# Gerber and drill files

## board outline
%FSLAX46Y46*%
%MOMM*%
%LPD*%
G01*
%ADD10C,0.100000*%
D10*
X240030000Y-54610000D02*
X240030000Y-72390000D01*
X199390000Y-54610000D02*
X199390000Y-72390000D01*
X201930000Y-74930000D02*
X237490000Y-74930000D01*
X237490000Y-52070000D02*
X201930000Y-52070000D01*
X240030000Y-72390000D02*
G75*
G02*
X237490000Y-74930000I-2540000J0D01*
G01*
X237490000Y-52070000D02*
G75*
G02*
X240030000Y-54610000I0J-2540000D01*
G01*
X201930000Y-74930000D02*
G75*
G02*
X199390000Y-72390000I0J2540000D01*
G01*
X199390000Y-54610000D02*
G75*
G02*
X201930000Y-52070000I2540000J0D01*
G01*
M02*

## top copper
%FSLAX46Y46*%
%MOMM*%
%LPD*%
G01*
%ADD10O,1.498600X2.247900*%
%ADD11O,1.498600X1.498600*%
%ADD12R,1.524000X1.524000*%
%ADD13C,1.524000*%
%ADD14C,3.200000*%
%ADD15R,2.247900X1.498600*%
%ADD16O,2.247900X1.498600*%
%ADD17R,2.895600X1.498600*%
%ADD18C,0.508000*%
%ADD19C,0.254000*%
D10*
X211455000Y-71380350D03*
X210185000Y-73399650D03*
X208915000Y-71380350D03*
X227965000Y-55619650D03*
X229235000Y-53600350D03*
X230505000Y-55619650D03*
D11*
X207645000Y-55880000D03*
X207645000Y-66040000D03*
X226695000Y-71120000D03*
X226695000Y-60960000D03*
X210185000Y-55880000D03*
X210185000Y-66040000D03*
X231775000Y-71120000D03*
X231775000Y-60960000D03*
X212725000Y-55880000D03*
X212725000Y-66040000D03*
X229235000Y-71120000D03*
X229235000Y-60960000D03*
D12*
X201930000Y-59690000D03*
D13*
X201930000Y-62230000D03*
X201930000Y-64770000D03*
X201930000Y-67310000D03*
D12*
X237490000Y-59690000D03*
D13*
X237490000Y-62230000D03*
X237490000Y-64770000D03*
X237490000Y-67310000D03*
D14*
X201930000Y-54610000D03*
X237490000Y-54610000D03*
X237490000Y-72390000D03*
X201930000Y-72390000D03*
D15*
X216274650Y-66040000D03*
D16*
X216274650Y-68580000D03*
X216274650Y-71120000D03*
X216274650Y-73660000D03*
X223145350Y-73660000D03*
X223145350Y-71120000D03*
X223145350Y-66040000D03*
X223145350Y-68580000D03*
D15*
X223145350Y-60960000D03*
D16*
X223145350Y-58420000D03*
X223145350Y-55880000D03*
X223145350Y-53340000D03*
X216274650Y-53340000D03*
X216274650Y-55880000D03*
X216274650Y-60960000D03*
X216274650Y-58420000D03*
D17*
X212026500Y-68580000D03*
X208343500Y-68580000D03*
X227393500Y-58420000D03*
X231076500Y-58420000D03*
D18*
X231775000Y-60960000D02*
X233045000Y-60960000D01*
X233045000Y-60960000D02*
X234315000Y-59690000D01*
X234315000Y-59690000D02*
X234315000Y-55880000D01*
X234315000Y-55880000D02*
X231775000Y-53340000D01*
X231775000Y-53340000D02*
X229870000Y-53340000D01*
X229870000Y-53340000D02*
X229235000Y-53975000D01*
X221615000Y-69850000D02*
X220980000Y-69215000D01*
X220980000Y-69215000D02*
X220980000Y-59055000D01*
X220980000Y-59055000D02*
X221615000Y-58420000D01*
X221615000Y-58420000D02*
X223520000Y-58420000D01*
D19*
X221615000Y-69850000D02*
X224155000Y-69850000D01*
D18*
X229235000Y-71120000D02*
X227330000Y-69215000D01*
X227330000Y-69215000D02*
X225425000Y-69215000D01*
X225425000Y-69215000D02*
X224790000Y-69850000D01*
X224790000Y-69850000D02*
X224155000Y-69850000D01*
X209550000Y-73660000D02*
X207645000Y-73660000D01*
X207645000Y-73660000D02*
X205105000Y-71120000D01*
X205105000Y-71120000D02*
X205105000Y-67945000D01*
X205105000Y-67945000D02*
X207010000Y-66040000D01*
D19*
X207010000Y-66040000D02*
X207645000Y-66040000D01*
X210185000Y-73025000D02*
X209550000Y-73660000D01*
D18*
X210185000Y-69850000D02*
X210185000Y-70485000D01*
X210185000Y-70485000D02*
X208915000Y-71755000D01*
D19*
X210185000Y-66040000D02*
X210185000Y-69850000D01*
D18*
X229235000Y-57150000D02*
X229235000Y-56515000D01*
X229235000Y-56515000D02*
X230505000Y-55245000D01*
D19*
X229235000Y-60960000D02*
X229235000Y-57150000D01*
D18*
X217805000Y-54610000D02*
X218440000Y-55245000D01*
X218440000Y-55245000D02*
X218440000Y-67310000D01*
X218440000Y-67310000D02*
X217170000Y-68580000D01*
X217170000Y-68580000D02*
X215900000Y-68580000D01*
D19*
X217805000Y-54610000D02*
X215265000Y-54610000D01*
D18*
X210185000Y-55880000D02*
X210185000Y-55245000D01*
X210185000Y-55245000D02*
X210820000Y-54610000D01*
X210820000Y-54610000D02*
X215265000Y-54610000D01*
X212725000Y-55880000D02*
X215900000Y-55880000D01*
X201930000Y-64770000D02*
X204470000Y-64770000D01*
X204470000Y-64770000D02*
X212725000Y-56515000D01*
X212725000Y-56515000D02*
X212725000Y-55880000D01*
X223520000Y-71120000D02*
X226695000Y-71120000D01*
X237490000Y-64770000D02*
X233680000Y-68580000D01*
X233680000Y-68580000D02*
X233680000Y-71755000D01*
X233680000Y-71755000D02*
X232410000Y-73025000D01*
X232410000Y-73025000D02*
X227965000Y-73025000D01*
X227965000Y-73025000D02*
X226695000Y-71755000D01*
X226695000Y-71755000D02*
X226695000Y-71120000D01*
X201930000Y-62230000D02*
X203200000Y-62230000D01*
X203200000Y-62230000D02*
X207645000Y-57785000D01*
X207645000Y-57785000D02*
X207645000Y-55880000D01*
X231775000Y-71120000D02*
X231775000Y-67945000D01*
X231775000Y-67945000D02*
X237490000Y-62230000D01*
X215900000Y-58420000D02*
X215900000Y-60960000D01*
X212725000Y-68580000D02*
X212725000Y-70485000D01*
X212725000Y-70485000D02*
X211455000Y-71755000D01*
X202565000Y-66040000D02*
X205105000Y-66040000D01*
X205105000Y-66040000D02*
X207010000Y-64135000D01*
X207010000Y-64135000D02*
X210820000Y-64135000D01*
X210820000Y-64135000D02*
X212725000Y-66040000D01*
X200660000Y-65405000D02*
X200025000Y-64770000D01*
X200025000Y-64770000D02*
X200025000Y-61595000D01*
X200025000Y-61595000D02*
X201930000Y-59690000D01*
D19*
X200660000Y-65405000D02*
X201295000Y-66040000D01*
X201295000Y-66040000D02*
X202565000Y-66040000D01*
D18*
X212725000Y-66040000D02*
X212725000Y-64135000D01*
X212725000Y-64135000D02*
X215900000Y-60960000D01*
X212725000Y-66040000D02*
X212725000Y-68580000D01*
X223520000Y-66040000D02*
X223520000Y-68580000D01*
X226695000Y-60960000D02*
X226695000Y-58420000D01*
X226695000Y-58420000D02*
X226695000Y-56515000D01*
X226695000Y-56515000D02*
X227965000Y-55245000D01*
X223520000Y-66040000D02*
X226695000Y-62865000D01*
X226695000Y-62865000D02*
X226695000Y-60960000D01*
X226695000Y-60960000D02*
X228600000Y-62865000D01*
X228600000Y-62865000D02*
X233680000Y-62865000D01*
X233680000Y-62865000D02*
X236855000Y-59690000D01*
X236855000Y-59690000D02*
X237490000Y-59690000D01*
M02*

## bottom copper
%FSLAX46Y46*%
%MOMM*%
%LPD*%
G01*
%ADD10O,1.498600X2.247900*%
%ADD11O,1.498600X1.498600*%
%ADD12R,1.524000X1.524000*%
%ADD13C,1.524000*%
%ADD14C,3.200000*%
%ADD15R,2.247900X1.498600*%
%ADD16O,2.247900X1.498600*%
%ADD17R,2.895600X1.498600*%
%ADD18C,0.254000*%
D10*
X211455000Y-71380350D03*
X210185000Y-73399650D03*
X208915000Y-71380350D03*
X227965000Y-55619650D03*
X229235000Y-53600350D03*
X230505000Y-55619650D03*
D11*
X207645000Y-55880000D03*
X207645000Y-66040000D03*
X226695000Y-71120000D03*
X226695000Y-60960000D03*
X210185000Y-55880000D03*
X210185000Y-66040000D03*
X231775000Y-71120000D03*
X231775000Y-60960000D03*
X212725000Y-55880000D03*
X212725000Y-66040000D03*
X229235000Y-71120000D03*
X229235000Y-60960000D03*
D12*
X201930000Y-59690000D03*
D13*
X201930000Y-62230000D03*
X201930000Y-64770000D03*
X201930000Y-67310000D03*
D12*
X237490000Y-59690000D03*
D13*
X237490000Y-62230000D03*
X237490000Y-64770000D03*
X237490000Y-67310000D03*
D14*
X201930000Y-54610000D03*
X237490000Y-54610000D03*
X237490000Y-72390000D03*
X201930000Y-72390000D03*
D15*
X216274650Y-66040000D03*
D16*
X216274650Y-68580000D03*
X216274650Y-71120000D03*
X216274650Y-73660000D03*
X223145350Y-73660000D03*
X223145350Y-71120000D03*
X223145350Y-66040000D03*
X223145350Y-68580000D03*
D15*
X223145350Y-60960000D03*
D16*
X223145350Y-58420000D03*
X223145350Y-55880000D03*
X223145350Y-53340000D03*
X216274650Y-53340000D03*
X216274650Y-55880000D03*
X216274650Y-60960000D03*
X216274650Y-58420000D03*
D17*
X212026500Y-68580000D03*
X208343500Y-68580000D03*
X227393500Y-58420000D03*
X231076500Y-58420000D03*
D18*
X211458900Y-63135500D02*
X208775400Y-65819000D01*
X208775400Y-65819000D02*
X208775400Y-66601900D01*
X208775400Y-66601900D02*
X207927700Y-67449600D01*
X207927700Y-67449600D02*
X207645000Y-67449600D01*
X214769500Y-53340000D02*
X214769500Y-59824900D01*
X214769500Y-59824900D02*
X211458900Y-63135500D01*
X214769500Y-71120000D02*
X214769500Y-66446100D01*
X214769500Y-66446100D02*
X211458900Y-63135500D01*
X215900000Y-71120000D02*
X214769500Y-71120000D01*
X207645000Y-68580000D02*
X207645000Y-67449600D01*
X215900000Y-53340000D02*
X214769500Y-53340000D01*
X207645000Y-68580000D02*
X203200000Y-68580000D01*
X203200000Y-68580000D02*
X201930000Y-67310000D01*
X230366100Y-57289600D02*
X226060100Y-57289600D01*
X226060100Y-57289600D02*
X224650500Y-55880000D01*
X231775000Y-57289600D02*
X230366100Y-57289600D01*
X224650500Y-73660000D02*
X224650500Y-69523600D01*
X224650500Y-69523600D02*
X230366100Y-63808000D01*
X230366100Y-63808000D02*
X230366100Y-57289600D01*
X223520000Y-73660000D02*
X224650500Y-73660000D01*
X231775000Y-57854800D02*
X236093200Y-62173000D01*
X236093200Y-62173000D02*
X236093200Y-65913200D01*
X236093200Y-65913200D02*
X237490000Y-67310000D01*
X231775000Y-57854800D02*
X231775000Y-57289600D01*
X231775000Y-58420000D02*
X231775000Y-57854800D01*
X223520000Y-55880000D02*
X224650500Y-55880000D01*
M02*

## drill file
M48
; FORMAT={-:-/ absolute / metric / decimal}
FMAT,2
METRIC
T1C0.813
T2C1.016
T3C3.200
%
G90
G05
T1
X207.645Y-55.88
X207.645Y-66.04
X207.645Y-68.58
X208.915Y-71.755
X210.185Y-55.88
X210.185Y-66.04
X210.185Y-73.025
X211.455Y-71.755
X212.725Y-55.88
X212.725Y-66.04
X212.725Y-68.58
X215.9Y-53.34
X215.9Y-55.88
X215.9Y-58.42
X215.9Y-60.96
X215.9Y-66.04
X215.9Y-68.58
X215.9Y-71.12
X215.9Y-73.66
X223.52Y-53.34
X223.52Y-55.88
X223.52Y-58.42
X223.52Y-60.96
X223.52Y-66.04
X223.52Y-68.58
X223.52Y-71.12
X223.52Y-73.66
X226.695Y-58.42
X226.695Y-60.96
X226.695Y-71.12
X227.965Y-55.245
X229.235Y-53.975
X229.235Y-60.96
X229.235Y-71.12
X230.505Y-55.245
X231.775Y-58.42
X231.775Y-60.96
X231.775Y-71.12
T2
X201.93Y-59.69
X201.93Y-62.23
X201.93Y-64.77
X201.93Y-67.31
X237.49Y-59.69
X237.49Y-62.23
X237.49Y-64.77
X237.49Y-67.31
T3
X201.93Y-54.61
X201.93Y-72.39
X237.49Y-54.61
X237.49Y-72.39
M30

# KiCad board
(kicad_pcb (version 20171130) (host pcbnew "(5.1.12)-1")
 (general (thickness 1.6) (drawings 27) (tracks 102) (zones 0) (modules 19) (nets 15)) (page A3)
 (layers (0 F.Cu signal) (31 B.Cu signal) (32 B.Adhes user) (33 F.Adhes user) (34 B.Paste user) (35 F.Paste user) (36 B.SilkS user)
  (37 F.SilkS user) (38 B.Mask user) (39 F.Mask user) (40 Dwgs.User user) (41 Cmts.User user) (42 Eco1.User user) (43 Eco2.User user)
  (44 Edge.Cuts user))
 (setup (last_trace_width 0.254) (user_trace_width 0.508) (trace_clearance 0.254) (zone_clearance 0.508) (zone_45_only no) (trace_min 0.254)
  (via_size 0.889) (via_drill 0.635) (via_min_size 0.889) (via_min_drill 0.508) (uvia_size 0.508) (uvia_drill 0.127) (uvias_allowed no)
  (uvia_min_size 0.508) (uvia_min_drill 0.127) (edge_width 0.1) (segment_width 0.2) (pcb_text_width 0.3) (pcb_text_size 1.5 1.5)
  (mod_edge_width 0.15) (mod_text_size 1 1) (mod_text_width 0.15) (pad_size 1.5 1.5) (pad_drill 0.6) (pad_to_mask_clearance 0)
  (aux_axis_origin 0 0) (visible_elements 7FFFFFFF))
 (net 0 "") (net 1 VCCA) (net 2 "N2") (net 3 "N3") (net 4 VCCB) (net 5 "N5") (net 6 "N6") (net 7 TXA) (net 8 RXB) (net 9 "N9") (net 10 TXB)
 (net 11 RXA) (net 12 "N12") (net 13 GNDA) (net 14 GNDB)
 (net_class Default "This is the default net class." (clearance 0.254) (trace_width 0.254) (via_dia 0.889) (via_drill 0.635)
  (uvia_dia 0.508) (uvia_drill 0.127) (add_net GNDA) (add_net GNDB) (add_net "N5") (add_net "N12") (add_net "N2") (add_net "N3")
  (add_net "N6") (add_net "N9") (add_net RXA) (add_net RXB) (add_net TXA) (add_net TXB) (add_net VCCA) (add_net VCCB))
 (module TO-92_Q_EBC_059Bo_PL (layer F.Cu) (at 211.455 71.755)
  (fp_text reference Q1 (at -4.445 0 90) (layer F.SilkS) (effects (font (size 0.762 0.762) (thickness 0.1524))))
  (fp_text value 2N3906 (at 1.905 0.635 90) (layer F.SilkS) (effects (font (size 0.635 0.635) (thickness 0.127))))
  (pad 1 thru_hole oval (at 0 0) (size 1.4986 2.2479) (drill 0.8128 (offset 0 -0.37465)) (layers *.Cu *.Mask F.SilkS) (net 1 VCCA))
  (pad 2 thru_hole oval (at -1.27 1.27) (size 1.4986 2.2479) (drill 0.8128 (offset 0 0.37465)) (layers *.Cu *.Mask F.SilkS) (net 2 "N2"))
  (pad 3 thru_hole oval (at -2.54 0) (size 1.4986 2.2479) (drill 0.8128 (offset 0 -0.37465)) (layers *.Cu *.Mask F.SilkS) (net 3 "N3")))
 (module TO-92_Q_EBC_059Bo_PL (layer F.Cu) (at 227.965 55.245 180)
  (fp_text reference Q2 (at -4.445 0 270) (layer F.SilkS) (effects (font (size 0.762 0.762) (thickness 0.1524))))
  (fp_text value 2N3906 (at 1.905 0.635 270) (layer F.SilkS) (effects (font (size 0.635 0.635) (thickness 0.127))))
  (pad 1 thru_hole oval (at 0 0 180) (size 1.4986 2.2479) (drill 0.8128 (offset 0 -0.37465)) (layers *.Cu *.Mask F.SilkS) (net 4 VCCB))
  (pad 2 thru_hole oval (at -1.27 1.27 180) (size 1.4986 2.2479) (drill 0.8128 (offset 0 0.37465)) (layers *.Cu *.Mask F.SilkS) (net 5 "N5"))
  (pad 3 thru_hole oval (at -2.54 0 180) (size 1.4986 2.2479) (drill 0.8128 (offset 0 -0.37465)) (layers *.Cu *.Mask F.SilkS) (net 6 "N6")))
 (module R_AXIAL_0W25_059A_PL (layer F.Cu) (at 207.645 55.88 270) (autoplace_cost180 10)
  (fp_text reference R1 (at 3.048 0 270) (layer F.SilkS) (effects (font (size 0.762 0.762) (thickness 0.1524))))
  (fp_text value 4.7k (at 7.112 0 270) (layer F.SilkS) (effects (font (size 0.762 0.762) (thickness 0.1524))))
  (pad 1 thru_hole oval (at 0 0 270) (size 1.4986 1.4986) (drill 0.8128) (layers *.Cu *.Mask F.SilkS) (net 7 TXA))
  (pad 2 thru_hole oval (at 10.16 0 270) (size 1.4986 1.4986) (drill 0.8128) (layers *.Cu *.Mask F.SilkS) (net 2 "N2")))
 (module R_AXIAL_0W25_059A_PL (layer F.Cu) (at 226.695 71.12 90) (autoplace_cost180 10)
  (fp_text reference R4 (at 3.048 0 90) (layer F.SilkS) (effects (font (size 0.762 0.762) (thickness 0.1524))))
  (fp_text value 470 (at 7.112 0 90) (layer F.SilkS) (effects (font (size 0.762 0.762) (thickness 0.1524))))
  (pad 1 thru_hole oval (at 0 0 90) (size 1.4986 1.4986) (drill 0.8128) (layers *.Cu *.Mask F.SilkS) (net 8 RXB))
  (pad 2 thru_hole oval (at 10.16 0 90) (size 1.4986 1.4986) (drill 0.8128) (layers *.Cu *.Mask F.SilkS) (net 4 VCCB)))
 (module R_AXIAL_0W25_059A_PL (layer F.Cu) (at 210.185 55.88 270) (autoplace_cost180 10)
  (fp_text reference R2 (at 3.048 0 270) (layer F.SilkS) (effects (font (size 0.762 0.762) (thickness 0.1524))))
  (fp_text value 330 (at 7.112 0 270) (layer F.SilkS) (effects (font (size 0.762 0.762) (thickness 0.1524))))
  (pad 1 thru_hole oval (at 0 0 270) (size 1.4986 1.4986) (drill 0.8128) (layers *.Cu *.Mask F.SilkS) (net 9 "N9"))
  (pad 2 thru_hole oval (at 10.16 0 270) (size 1.4986 1.4986) (drill 0.8128) (layers *.Cu *.Mask F.SilkS) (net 3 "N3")))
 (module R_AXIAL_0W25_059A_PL (layer F.Cu) (at 231.775 71.12 90) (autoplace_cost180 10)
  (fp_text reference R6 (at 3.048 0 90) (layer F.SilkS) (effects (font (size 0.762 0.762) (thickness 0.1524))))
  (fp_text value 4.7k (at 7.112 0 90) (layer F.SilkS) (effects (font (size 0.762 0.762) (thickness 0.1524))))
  (pad 1 thru_hole oval (at 0 0 90) (size 1.4986 1.4986) (drill 0.8128) (layers *.Cu *.Mask F.SilkS) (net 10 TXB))
  (pad 2 thru_hole oval (at 10.16 0 90) (size 1.4986 1.4986) (drill 0.8128) (layers *.Cu *.Mask F.SilkS) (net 5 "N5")))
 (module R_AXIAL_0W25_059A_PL (layer F.Cu) (at 212.725 55.88 270) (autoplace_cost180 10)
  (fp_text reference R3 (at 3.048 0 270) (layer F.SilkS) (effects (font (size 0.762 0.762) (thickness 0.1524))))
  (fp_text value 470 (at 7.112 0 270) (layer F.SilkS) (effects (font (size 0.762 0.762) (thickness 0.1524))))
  (pad 1 thru_hole oval (at 0 0 270) (size 1.4986 1.4986) (drill 0.8128) (layers *.Cu *.Mask F.SilkS) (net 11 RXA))
  (pad 2 thru_hole oval (at 10.16 0 270) (size 1.4986 1.4986) (drill 0.8128) (layers *.Cu *.Mask F.SilkS) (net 1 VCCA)))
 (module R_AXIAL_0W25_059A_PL (layer F.Cu) (at 229.235 71.12 90) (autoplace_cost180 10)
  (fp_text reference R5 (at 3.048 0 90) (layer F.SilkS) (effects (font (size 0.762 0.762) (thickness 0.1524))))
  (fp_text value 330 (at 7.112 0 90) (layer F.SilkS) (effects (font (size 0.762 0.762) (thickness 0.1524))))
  (pad 1 thru_hole oval (at 0 0 90) (size 1.4986 1.4986) (drill 0.8128) (layers *.Cu *.Mask F.SilkS) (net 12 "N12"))
  (pad 2 thru_hole oval (at 10.16 0 90) (size 1.4986 1.4986) (drill 0.8128) (layers *.Cu *.Mask F.SilkS) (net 6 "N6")))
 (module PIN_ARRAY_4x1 (layer F.Cu) (at 201.93 63.5 270)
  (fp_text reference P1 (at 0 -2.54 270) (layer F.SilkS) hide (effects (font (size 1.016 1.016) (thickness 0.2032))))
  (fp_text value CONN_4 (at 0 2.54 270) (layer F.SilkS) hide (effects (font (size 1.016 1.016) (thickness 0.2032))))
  (pad 1 thru_hole rect (at -3.81 0 270) (size 1.524 1.524) (drill 1.016) (layers *.Cu *.Mask F.SilkS) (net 1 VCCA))
  (pad 2 thru_hole circle (at -1.27 0 270) (size 1.524 1.524) (drill 1.016) (layers *.Cu *.Mask F.SilkS) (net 7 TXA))
  (pad 3 thru_hole circle (at 1.27 0 270) (size 1.524 1.524) (drill 1.016) (layers *.Cu *.Mask F.SilkS) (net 11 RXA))
  (pad 4 thru_hole circle (at 3.81 0 270) (size 1.524 1.524) (drill 1.016) (layers *.Cu *.Mask F.SilkS) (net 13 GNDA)))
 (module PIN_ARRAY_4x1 (layer F.Cu) (at 237.49 63.5 270)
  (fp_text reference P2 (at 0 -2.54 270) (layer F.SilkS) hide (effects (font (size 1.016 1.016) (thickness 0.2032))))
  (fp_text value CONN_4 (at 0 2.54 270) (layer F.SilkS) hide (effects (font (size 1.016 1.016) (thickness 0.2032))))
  (pad 1 thru_hole rect (at -3.81 0 270) (size 1.524 1.524) (drill 1.016) (layers *.Cu *.Mask F.SilkS) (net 4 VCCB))
  (pad 2 thru_hole circle (at -1.27 0 270) (size 1.524 1.524) (drill 1.016) (layers *.Cu *.Mask F.SilkS) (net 10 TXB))
  (pad 3 thru_hole circle (at 1.27 0 270) (size 1.524 1.524) (drill 1.016) (layers *.Cu *.Mask F.SilkS) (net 8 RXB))
  (pad 4 thru_hole circle (at 3.81 0 270) (size 1.524 1.524) (drill 1.016) (layers *.Cu *.Mask F.SilkS) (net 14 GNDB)))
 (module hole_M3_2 (layer F.Cu) (at 201.93 54.61)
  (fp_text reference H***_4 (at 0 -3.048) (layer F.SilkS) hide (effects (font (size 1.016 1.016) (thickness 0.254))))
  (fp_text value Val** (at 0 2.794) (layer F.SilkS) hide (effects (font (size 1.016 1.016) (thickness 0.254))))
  (pad 1 thru_hole circle (at 0 0) (size 3.2 3.2) (drill 3.2) (layers *.Cu *.Mask F.SilkS)))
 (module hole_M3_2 (layer F.Cu) (at 237.49 54.61)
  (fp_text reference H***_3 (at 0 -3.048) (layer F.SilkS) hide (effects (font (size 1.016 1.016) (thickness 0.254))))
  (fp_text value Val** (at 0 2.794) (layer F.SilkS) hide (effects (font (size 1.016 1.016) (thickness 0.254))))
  (pad 1 thru_hole circle (at 0 0) (size 3.2 3.2) (drill 3.2) (layers *.Cu *.Mask F.SilkS)))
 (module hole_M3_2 (layer F.Cu) (at 237.49 72.39)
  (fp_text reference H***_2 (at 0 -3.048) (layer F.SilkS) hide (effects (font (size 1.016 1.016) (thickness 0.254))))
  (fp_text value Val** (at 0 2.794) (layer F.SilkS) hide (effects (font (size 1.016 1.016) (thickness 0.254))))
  (pad 1 thru_hole circle (at 0 0) (size 3.2 3.2) (drill 3.2) (layers *.Cu *.Mask F.SilkS)))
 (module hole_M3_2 (layer F.Cu) (at 201.93 72.39)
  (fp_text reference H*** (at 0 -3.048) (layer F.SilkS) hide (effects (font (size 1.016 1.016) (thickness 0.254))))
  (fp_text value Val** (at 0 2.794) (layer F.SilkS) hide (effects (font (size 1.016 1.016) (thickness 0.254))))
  (pad 1 thru_hole circle (at 0 0) (size 3.2 3.2) (drill 3.2) (layers *.Cu *.Mask F.SilkS)))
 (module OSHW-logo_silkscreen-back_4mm (layer F.Cu) (at 210.185 60.325)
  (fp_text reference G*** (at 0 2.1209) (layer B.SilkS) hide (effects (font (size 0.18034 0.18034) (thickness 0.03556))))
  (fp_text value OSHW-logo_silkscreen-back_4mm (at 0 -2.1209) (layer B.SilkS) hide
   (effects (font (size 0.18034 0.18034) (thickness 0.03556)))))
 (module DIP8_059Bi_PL (layer F.Cu) (at 215.9 66.04 270)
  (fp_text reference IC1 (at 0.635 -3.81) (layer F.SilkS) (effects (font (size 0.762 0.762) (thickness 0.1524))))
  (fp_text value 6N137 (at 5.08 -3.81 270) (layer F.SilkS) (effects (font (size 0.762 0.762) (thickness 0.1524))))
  (pad 1 thru_hole rect (at 0 0 270) (size 1.4986 2.2479) (drill 0.8128 (offset 0 -0.37465)) (layers *.Cu *.Mask F.SilkS))
  (pad 2 thru_hole oval (at 2.54 0 270) (size 1.4986 2.2479) (drill 0.8128 (offset 0 -0.37465)) (layers *.Cu *.Mask F.SilkS) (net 9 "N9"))
  (pad 3 thru_hole oval (at 5.08 0 270) (size 1.4986 2.2479) (drill 0.8128 (offset 0 -0.37465)) (layers *.Cu *.Mask F.SilkS) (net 13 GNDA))
  (pad 4 thru_hole oval (at 7.62 0 270) (size 1.4986 2.2479) (drill 0.8128 (offset 0 -0.37465)) (layers *.Cu *.Mask F.SilkS))
  (pad 5 thru_hole oval (at 7.62 -7.62 270) (size 1.4986 2.2479) (drill 0.8128 (offset 0 0.37465)) (layers *.Cu *.Mask F.SilkS)
   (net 14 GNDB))
  (pad 6 thru_hole oval (at 5.08 -7.62 270) (size 1.4986 2.2479) (drill 0.8128 (offset 0 0.37465)) (layers *.Cu *.Mask F.SilkS) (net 8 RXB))
  (pad 8 thru_hole oval (at 0 -7.62 270) (size 1.4986 2.2479) (drill 0.8128 (offset 0 0.37465)) (layers *.Cu *.Mask F.SilkS) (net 4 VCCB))
  (pad 7 thru_hole oval (at 2.54 -7.62 270) (size 1.4986 2.2479) (drill 0.8128 (offset 0 0.37465)) (layers *.Cu *.Mask F.SilkS) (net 4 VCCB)))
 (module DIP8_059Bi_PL (layer F.Cu) (at 223.52 60.96 90)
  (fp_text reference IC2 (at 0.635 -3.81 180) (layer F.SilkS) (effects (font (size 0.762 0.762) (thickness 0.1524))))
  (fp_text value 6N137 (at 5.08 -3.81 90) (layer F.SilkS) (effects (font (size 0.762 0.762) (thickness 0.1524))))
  (pad 1 thru_hole rect (at 0 0 90) (size 1.4986 2.2479) (drill 0.8128 (offset 0 -0.37465)) (layers *.Cu *.Mask F.SilkS))
  (pad 2 thru_hole oval (at 2.54 0 90) (size 1.4986 2.2479) (drill 0.8128 (offset 0 -0.37465)) (layers *.Cu *.Mask F.SilkS) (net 12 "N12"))
  (pad 3 thru_hole oval (at 5.08 0 90) (size 1.4986 2.2479) (drill 0.8128 (offset 0 -0.37465)) (layers *.Cu *.Mask F.SilkS) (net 14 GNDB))
  (pad 4 thru_hole oval (at 7.62 0 90) (size 1.4986 2.2479) (drill 0.8128 (offset 0 -0.37465)) (layers *.Cu *.Mask F.SilkS))
  (pad 5 thru_hole oval (at 7.62 -7.62 90) (size 1.4986 2.2479) (drill 0.8128 (offset 0 0.37465)) (layers *.Cu *.Mask F.SilkS) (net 13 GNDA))
  (pad 6 thru_hole oval (at 5.08 -7.62 90) (size 1.4986 2.2479) (drill 0.8128 (offset 0 0.37465)) (layers *.Cu *.Mask F.SilkS) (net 11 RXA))
  (pad 8 thru_hole oval (at 0 -7.62 90) (size 1.4986 2.2479) (drill 0.8128 (offset 0 0.37465)) (layers *.Cu *.Mask F.SilkS) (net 1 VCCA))
  (pad 7 thru_hole oval (at 2.54 -7.62 90) (size 1.4986 2.2479) (drill 0.8128 (offset 0 0.37465)) (layers *.Cu *.Mask F.SilkS) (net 1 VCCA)))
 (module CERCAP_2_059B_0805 (layer F.Cu) (at 210.185 68.58 180)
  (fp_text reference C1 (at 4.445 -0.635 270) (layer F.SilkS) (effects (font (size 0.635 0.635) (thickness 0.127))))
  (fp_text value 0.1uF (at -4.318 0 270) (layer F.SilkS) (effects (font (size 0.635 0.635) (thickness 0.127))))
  (pad 1 thru_hole rect (at -2.54 0 180) (size 2.8956 1.4986) (drill 0.8128 (offset 0.6985 0)) (layers *.Cu *.Mask F.SilkS) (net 1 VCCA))
  (pad 2 thru_hole rect (at 2.54 0 180) (size 2.8956 1.4986) (drill 0.8128 (offset -0.6985 0)) (layers *.Cu *.Mask F.SilkS) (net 13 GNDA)))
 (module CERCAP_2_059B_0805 (layer F.Cu) (at 229.235 58.42)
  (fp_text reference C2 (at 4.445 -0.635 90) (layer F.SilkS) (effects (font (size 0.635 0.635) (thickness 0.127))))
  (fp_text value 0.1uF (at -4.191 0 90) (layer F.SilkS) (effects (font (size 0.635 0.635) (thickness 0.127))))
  (pad 1 thru_hole rect (at -2.54 0) (size 2.8956 1.4986) (drill 0.8128 (offset 0.6985 0)) (layers *.Cu *.Mask F.SilkS) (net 4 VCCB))
  (pad 2 thru_hole rect (at 2.54 0) (size 2.8956 1.4986) (drill 0.8128 (offset -0.6985 0)) (layers *.Cu *.Mask F.SilkS) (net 14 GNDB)))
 (gr_line (start 240.03 54.61) (end 240.03 72.39) (angle 90) (layer Edge.Cuts) (width 0.1))
 (gr_line (start 199.39 54.61) (end 199.39 72.39) (angle 90) (layer Edge.Cuts) (width 0.1))
 (gr_line (start 201.93 74.93) (end 237.49 74.93) (angle 90) (layer Edge.Cuts) (width 0.1))
 (gr_line (start 237.49 52.07) (end 201.93 52.07) (angle 90) (layer Edge.Cuts) (width 0.1))
 (gr_arc (start 237.49 72.39) (end 240.03 72.39) (angle 90) (layer Edge.Cuts) (width 0.1))
 (gr_arc (start 237.49 54.61) (end 237.49 52.07) (angle 90) (layer Edge.Cuts) (width 0.1))
 (gr_arc (start 201.93 72.39) (end 201.93 74.93) (angle 90) (layer Edge.Cuts) (width 0.1))
 (gr_arc (start 201.93 54.61) (end 199.39 54.61) (angle 90) (layer Edge.Cuts) (width 0.1))
 (segment (start 211.4589 63.1355) (end 208.7754 65.819) (width 0.254) (layer B.Cu) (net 13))
 (segment (start 208.7754 65.819) (end 208.7754 66.6019) (width 0.254) (layer B.Cu) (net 13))
 (segment (start 208.7754 66.6019) (end 207.9277 67.4496) (width 0.254) (layer B.Cu) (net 13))
 (segment (start 207.9277 67.4496) (end 207.645 67.4496) (width 0.254) (layer B.Cu) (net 13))
 (segment (start 214.7695 53.34) (end 214.7695 59.8249) (width 0.254) (layer B.Cu) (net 13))
 (segment (start 214.7695 59.8249) (end 211.4589 63.1355) (width 0.254) (layer B.Cu) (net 13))
 (segment (start 214.7695 71.12) (end 214.7695 66.4461) (width 0.254) (layer B.Cu) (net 13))
 (segment (start 214.7695 66.4461) (end 211.4589 63.1355) (width 0.254) (layer B.Cu) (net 13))
 (segment (start 215.9 71.12) (end 214.7695 71.12) (width 0.254) (layer B.Cu) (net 13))
 (segment (start 207.645 68.58) (end 207.645 67.4496) (width 0.254) (layer B.Cu) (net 13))
 (segment (start 215.9 53.34) (end 214.7695 53.34) (width 0.254) (layer B.Cu) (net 13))
 (segment (start 207.645 68.58) (end 203.2 68.58) (width 0.254) (layer B.Cu) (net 13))
 (segment (start 203.2 68.58) (end 201.93 67.31) (width 0.254) (layer B.Cu) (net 13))
 (segment (start 230.3661 57.2896) (end 226.0601 57.2896) (width 0.254) (layer B.Cu) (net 14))
 (segment (start 226.0601 57.2896) (end 224.6505 55.88) (width 0.254) (layer B.Cu) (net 14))
 (segment (start 231.775 57.2896) (end 230.3661 57.2896) (width 0.254) (layer B.Cu) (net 14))
 (segment (start 224.6505 73.66) (end 224.6505 69.5236) (width 0.254) (layer B.Cu) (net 14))
 (segment (start 224.6505 69.5236) (end 230.3661 63.808) (width 0.254) (layer B.Cu) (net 14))
 (segment (start 230.3661 63.808) (end 230.3661 57.2896) (width 0.254) (layer B.Cu) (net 14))
 (segment (start 223.52 73.66) (end 224.6505 73.66) (width 0.254) (layer B.Cu) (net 14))
 (segment (start 231.775 57.8548) (end 236.0932 62.173) (width 0.254) (layer B.Cu) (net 14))
 (segment (start 236.0932 62.173) (end 236.0932 65.9132) (width 0.254) (layer B.Cu) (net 14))
 (segment (start 236.0932 65.9132) (end 237.49 67.31) (width 0.254) (layer B.Cu) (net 14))
 (segment (start 231.775 57.8548) (end 231.775 57.2896) (width 0.254) (layer B.Cu) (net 14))
 (segment (start 231.775 58.42) (end 231.775 57.8548) (width 0.254) (layer B.Cu) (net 14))
 (segment (start 223.52 55.88) (end 224.6505 55.88) (width 0.254) (layer B.Cu) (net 14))
 (segment (start 231.775 60.96) (end 233.045 60.96) (width 0.508) (layer F.Cu) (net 5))
 (segment (start 233.045 60.96) (end 234.315 59.69) (width 0.508) (layer F.Cu) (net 5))
 (segment (start 234.315 59.69) (end 234.315 55.88) (width 0.508) (layer F.Cu) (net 5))
 (segment (start 234.315 55.88) (end 231.775 53.34) (width 0.508) (layer F.Cu) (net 5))
 (segment (start 231.775 53.34) (end 229.87 53.34) (width 0.508) (layer F.Cu) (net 5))
 (segment (start 229.87 53.34) (end 229.235 53.975) (width 0.508) (layer F.Cu) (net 5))
 (segment (start 221.615 69.85) (end 220.98 69.215) (width 0.508) (layer F.Cu) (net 12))
 (segment (start 220.98 69.215) (end 220.98 59.055) (width 0.508) (layer F.Cu) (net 12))
 (segment (start 220.98 59.055) (end 221.615 58.42) (width 0.508) (layer F.Cu) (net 12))
 (segment (start 221.615 58.42) (end 223.52 58.42) (width 0.508) (layer F.Cu) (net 12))
 (segment (start 221.615 69.85) (end 224.155 69.85) (width 0.254) (layer F.Cu) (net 12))
 (segment (start 229.235 71.12) (end 227.33 69.215) (width 0.508) (layer F.Cu) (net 12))
 (segment (start 227.33 69.215) (end 225.425 69.215) (width 0.508) (layer F.Cu) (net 12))
 (segment (start 225.425 69.215) (end 224.79 69.85) (width 0.508) (layer F.Cu) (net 12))
 (segment (start 224.79 69.85) (end 224.155 69.85) (width 0.508) (layer F.Cu) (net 12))
 (segment (start 209.55 73.66) (end 207.645 73.66) (width 0.508) (layer F.Cu) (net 2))
 (segment (start 207.645 73.66) (end 205.105 71.12) (width 0.508) (layer F.Cu) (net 2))
 (segment (start 205.105 71.12) (end 205.105 67.945) (width 0.508) (layer F.Cu) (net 2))
 (segment (start 205.105 67.945) (end 207.01 66.04) (width 0.508) (layer F.Cu) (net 2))
 (segment (start 207.01 66.04) (end 207.645 66.04) (width 0.254) (layer F.Cu) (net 2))
 (segment (start 210.185 73.025) (end 209.55 73.66) (width 0.254) (layer F.Cu) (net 2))
 (segment (start 210.185 69.85) (end 210.185 70.485) (width 0.508) (layer F.Cu) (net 3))
 (segment (start 210.185 70.485) (end 208.915 71.755) (width 0.508) (layer F.Cu) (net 3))
 (segment (start 210.185 66.04) (end 210.185 69.85) (width 0.254) (layer F.Cu) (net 3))
 (segment (start 229.235 57.15) (end 229.235 56.515) (width 0.508) (layer F.Cu) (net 6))
 (segment (start 229.235 56.515) (end 230.505 55.245) (width 0.508) (layer F.Cu) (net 6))
 (segment (start 229.235 60.96) (end 229.235 57.15) (width 0.254) (layer F.Cu) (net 6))
 (segment (start 217.805 54.61) (end 218.44 55.245) (width 0.508) (layer F.Cu) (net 9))
 (segment (start 218.44 55.245) (end 218.44 67.31) (width 0.508) (layer F.Cu) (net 9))
 (segment (start 218.44 67.31) (end 217.17 68.58) (width 0.508) (layer F.Cu) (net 9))
 (segment (start 217.17 68.58) (end 215.9 68.58) (width 0.508) (layer F.Cu) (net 9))
 (segment (start 217.805 54.61) (end 215.265 54.61) (width 0.254) (layer F.Cu) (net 9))
 (segment (start 210.185 55.88) (end 210.185 55.245) (width 0.508) (layer F.Cu) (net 9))
 (segment (start 210.185 55.245) (end 210.82 54.61) (width 0.508) (layer F.Cu) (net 9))
 (segment (start 210.82 54.61) (end 215.265 54.61) (width 0.508) (layer F.Cu) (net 9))
 (segment (start 212.725 55.88) (end 215.9 55.88) (width 0.508) (layer F.Cu) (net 11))
 (segment (start 201.93 64.77) (end 204.47 64.77) (width 0.508) (layer F.Cu) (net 11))
 (segment (start 204.47 64.77) (end 212.725 56.515) (width 0.508) (layer F.Cu) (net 11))
 (segment (start 212.725 56.515) (end 212.725 55.88) (width 0.508) (layer F.Cu) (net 11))
 (segment (start 223.52 71.12) (end 226.695 71.12) (width 0.508) (layer F.Cu) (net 8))
 (segment (start 237.49 64.77) (end 233.68 68.58) (width 0.508) (layer F.Cu) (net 8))
 (segment (start 233.68 68.58) (end 233.68 71.755) (width 0.508) (layer F.Cu) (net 8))
 (segment (start 233.68 71.755) (end 232.41 73.025) (width 0.508) (layer F.Cu) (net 8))
 (segment (start 232.41 73.025) (end 227.965 73.025) (width 0.508) (layer F.Cu) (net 8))
 (segment (start 227.965 73.025) (end 226.695 71.755) (width 0.508) (layer F.Cu) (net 8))
 (segment (start 226.695 71.755) (end 226.695 71.12) (width 0.508) (layer F.Cu) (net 8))
 (segment (start 201.93 62.23) (end 203.2 62.23) (width 0.508) (layer F.Cu) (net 7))
 (segment (start 203.2 62.23) (end 207.645 57.785) (width 0.508) (layer F.Cu) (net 7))
 (segment (start 207.645 57.785) (end 207.645 55.88) (width 0.508) (layer F.Cu) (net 7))
 (segment (start 231.775 71.12) (end 231.775 67.945) (width 0.508) (layer F.Cu) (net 10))
 (segment (start 231.775 67.945) (end 237.49 62.23) (width 0.508) (layer F.Cu) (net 10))
 (segment (start 215.9 58.42) (end 215.9 60.96) (width 0.508) (layer F.Cu) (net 1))
 (segment (start 212.725 68.58) (end 212.725 70.485) (width 0.508) (layer F.Cu) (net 1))
 (segment (start 212.725 70.485) (end 211.455 71.755) (width 0.508) (layer F.Cu) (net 1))
 (segment (start 202.565 66.04) (end 205.105 66.04) (width 0.508) (layer F.Cu) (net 1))
 (segment (start 205.105 66.04) (end 207.01 64.135) (width 0.508) (layer F.Cu) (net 1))
 (segment (start 207.01 64.135) (end 210.82 64.135) (width 0.508) (layer F.Cu) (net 1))
 (segment (start 210.82 64.135) (end 212.725 66.04) (width 0.508) (layer F.Cu) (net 1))
 (segment (start 200.66 65.405) (end 200.025 64.77) (width 0.508) (layer F.Cu) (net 1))
 (segment (start 200.025 64.77) (end 200.025 61.595) (width 0.508) (layer F.Cu) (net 1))
 (segment (start 200.025 61.595) (end 201.93 59.69) (width 0.508) (layer F.Cu) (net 1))
 (segment (start 200.66 65.405) (end 201.295 66.04) (width 0.254) (layer F.Cu) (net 1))
 (segment (start 201.295 66.04) (end 202.565 66.04) (width 0.254) (layer F.Cu) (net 1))
 (segment (start 212.725 66.04) (end 212.725 64.135) (width 0.508) (layer F.Cu) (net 1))
 (segment (start 212.725 64.135) (end 215.9 60.96) (width 0.508) (layer F.Cu) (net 1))
 (segment (start 212.725 66.04) (end 212.725 68.58) (width 0.508) (layer F.Cu) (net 1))
 (segment (start 223.52 66.04) (end 223.52 68.58) (width 0.508) (layer F.Cu) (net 4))
 (segment (start 226.695 60.96) (end 226.695 58.42) (width 0.508) (layer F.Cu) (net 4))
 (segment (start 226.695 58.42) (end 226.695 56.515) (width 0.508) (layer F.Cu) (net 4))
 (segment (start 226.695 56.515) (end 227.965 55.245) (width 0.508) (layer F.Cu) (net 4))
 (segment (start 223.52 66.04) (end 226.695 62.865) (width 0.508) (layer F.Cu) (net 4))
 (segment (start 226.695 62.865) (end 226.695 60.96) (width 0.508) (layer F.Cu) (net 4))
 (segment (start 226.695 60.96) (end 228.6 62.865) (width 0.508) (layer F.Cu) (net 4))
 (segment (start 228.6 62.865) (end 233.68 62.865) (width 0.508) (layer F.Cu) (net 4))
 (segment (start 233.68 62.865) (end 236.855 59.69) (width 0.508) (layer F.Cu) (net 4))
 (segment (start 236.855 59.69) (end 237.49 59.69) (width 0.508) (layer F.Cu) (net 4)))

